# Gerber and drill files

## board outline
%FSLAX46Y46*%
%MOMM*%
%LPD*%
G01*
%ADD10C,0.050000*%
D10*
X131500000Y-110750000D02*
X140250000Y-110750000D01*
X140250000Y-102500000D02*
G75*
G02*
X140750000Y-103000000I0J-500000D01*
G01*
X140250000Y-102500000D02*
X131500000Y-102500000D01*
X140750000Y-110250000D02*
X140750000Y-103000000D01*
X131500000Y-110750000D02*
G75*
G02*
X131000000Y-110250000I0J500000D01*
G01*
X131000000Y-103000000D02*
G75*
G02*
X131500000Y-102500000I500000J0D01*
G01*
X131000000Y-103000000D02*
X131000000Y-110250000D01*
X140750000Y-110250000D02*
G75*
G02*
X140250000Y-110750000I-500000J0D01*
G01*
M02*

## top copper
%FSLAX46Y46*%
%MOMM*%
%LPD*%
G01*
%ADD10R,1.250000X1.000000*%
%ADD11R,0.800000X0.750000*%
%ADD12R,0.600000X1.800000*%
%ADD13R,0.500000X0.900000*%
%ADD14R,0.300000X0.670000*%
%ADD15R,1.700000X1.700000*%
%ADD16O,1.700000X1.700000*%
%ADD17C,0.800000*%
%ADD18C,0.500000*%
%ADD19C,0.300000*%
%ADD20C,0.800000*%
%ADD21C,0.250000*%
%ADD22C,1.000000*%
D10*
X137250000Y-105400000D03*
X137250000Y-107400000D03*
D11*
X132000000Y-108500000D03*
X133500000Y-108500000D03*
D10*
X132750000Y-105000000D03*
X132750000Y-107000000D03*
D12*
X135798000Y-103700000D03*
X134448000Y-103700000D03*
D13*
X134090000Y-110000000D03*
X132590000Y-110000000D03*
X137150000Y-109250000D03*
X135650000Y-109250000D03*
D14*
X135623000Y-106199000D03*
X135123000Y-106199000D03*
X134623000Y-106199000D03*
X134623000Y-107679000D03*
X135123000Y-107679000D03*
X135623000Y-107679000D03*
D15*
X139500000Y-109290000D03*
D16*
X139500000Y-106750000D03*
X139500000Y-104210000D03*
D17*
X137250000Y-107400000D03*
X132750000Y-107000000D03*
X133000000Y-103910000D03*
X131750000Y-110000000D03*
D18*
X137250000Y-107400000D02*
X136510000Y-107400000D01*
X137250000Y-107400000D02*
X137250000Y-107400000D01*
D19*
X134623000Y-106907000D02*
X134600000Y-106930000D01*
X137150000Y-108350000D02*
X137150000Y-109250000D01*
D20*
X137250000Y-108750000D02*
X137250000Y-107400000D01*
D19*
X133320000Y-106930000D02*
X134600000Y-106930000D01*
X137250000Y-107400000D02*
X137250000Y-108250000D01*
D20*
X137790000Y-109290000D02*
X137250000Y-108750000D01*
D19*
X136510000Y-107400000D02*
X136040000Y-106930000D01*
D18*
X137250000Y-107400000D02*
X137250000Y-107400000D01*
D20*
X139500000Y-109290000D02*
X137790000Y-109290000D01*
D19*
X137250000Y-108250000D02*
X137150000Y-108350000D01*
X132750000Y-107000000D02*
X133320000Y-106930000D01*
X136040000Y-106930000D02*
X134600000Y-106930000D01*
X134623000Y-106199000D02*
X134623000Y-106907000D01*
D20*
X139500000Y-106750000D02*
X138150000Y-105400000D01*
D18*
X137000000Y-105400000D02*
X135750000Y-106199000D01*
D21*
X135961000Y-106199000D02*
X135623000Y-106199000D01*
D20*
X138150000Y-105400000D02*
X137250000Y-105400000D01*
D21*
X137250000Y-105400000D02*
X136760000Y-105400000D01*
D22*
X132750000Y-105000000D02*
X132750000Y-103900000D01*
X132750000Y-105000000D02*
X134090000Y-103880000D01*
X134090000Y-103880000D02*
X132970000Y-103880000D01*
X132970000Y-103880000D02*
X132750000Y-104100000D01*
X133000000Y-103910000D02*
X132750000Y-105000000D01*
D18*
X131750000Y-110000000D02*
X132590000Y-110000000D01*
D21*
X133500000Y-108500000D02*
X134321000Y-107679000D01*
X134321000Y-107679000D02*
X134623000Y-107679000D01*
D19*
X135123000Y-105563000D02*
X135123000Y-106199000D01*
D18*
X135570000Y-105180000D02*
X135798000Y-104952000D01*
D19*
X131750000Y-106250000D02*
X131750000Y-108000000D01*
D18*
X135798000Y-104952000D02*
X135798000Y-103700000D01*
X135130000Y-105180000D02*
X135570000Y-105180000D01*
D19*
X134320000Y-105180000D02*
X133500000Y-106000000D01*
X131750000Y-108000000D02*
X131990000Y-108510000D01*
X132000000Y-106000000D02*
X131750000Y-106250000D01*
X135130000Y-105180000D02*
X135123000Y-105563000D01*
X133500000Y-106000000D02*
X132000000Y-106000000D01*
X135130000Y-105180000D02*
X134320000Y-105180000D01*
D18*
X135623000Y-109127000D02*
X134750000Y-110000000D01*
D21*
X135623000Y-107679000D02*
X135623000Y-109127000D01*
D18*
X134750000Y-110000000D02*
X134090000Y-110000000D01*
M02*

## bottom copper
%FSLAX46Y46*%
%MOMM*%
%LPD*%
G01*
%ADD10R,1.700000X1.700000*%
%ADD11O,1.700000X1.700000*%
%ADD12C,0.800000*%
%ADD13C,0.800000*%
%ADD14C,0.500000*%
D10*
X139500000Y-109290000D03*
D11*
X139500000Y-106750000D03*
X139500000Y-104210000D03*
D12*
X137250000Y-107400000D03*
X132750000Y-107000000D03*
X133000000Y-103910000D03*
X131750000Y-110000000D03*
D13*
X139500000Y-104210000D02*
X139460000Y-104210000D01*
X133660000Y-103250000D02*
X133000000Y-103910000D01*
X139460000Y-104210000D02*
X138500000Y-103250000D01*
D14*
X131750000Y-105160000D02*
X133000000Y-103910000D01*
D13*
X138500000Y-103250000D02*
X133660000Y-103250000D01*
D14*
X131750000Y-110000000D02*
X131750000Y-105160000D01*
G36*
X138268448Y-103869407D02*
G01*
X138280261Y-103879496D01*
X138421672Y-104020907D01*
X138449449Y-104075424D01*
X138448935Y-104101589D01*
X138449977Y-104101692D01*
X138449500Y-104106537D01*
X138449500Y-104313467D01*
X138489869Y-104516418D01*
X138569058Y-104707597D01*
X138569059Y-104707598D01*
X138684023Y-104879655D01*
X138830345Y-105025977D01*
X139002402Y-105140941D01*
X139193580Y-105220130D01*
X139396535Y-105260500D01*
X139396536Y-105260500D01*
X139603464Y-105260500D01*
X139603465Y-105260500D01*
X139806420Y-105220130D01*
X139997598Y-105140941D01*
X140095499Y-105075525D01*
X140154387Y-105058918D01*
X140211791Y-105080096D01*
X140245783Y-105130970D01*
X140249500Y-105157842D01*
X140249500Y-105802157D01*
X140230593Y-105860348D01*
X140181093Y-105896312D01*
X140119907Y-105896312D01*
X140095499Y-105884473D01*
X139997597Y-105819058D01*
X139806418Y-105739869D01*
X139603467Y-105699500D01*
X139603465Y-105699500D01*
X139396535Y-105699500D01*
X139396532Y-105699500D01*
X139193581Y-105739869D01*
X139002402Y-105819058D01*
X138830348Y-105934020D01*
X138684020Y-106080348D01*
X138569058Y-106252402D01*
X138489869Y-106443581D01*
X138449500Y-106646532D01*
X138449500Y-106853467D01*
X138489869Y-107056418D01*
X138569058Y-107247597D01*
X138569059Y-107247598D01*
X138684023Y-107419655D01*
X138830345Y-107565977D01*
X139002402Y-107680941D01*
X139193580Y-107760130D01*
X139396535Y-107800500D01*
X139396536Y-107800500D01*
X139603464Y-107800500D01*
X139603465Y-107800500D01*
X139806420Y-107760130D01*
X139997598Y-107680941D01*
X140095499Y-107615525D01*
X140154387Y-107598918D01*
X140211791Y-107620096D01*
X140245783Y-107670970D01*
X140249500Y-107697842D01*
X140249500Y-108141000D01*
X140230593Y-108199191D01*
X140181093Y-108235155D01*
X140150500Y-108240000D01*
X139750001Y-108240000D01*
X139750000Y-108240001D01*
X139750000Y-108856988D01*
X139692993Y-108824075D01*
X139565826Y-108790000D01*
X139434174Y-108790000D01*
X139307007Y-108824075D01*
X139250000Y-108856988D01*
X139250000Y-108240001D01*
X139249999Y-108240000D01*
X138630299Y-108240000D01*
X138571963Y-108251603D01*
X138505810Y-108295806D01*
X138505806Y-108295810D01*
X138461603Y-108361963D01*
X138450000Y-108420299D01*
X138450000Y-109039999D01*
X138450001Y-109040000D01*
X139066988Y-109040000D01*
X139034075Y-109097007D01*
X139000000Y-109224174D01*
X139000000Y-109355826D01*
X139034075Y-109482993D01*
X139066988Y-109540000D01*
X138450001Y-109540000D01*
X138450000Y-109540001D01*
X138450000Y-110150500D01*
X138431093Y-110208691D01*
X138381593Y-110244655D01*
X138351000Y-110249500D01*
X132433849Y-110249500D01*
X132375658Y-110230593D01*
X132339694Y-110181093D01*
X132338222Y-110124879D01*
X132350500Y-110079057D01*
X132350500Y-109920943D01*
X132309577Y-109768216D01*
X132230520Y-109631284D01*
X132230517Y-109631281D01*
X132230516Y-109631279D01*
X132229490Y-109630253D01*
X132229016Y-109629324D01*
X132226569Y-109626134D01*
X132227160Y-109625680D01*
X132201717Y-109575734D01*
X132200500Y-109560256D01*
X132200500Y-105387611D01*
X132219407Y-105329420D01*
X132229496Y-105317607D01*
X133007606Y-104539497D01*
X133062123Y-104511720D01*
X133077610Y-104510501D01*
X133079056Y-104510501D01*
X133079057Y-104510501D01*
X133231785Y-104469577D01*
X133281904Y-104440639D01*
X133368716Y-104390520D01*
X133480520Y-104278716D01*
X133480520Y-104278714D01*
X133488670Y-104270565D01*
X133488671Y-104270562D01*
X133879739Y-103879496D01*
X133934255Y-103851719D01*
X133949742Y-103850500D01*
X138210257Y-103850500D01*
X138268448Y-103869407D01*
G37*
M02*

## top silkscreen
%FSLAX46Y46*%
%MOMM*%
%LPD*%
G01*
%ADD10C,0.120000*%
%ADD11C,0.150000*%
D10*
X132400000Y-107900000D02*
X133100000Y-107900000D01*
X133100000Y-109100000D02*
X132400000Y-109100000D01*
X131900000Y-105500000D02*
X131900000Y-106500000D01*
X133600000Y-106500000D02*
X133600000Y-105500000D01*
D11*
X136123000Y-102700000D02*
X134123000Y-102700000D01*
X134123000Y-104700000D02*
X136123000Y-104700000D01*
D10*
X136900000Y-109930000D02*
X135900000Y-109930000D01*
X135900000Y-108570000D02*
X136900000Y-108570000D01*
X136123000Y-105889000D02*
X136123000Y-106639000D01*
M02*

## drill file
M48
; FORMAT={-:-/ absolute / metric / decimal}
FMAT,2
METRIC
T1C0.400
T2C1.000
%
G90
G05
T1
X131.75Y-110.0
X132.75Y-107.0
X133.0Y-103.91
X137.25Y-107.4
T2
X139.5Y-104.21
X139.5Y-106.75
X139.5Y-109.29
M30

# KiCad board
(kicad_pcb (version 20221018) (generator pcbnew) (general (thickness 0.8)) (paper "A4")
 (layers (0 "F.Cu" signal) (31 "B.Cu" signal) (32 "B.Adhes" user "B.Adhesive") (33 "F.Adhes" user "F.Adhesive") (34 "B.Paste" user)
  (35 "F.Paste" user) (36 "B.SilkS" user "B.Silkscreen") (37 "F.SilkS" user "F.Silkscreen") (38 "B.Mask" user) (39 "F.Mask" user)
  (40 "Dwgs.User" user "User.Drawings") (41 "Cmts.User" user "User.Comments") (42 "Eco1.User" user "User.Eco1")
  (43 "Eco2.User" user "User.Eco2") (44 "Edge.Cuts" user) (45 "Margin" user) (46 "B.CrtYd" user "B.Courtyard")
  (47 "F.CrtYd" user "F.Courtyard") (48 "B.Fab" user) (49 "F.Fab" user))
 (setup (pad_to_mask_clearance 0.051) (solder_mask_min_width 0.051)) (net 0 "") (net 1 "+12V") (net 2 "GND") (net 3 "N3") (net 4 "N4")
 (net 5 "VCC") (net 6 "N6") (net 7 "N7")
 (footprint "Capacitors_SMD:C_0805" (layer "F.Cu") (at 137.25 106.4 -90)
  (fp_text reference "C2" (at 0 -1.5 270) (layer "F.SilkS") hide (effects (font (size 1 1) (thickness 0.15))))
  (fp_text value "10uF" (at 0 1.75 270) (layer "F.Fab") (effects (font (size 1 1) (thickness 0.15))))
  (pad "1" smd rect (at -1 0 270) (size 1 1.25) (layers "F.Cu" "F.Paste" "F.Mask") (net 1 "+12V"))
  (pad "2" smd rect (at 1 0 270) (size 1 1.25) (layers "F.Cu" "F.Paste" "F.Mask") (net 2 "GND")))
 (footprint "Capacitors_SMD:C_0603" (layer "F.Cu") (at 132.75 108.5)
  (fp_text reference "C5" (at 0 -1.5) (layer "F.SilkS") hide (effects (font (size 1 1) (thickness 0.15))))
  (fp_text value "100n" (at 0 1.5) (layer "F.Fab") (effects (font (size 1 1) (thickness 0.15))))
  (fp_line (start -0.35 -0.6) (end 0.35 -0.6) (stroke (width 0.12) (type solid)) (layer "F.SilkS"))
  (fp_line (start 0.35 0.6) (end -0.35 0.6) (stroke (width 0.12) (type solid)) (layer "F.SilkS"))
  (pad "1" smd rect (at -0.75 0) (size 0.8 0.75) (layers "F.Cu" "F.Paste" "F.Mask") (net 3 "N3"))
  (pad "2" smd rect (at 0.75 0) (size 0.8 0.75) (layers "F.Cu" "F.Paste" "F.Mask") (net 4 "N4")))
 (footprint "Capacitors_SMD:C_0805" (layer "F.Cu") (at 132.75 106 -90)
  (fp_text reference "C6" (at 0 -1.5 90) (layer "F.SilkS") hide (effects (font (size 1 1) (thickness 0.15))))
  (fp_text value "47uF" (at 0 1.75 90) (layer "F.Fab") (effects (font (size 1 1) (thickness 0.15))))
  (fp_line (start -0.5 0.85) (end 0.5 0.85) (stroke (width 0.12) (type solid)) (layer "F.SilkS"))
  (fp_line (start 0.5 -0.85) (end -0.5 -0.85) (stroke (width 0.12) (type solid)) (layer "F.SilkS"))
  (pad "1" smd rect (at -1 0 270) (size 1 1.25) (layers "F.Cu" "F.Paste" "F.Mask") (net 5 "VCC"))
  (pad "2" smd rect (at 1 0 270) (size 1 1.25) (layers "F.Cu" "F.Paste" "F.Mask") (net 2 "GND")))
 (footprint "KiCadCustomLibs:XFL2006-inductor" (layer "F.Cu") (at 135.123 103.7 180)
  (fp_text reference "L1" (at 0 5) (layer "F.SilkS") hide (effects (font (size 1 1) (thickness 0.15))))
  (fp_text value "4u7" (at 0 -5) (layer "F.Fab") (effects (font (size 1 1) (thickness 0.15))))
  (fp_line (start -1 1) (end 1 1) (stroke (width 0.15) (type solid)) (layer "F.SilkS"))
  (fp_line (start 1 -1) (end -1 -1) (stroke (width 0.15) (type solid)) (layer "F.SilkS"))
  (pad "1" smd rect (at -0.675 0 180) (size 0.6 1.8) (layers "F.Cu" "F.Paste" "F.Mask") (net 3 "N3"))
  (pad "2" smd rect (at 0.675 0 180) (size 0.6 1.8) (layers "F.Cu" "F.Paste" "F.Mask") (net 5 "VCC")))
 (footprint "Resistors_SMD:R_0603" (layer "F.Cu") (at 133.34 110 180)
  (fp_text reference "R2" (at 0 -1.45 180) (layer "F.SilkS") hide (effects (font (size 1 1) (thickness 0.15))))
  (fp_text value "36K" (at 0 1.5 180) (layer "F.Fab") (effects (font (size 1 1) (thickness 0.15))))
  (pad "1" smd rect (at -0.75 0 180) (size 0.5 0.9) (layers "F.Cu" "F.Paste" "F.Mask") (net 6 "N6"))
  (pad "2" smd rect (at 0.75 0 180) (size 0.5 0.9) (layers "F.Cu" "F.Paste" "F.Mask") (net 5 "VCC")))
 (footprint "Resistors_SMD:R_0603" (layer "F.Cu") (at 136.4 109.25 180)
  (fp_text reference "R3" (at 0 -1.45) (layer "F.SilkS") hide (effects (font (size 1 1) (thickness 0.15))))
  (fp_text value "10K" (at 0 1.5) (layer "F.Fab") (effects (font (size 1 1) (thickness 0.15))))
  (fp_line (start -0.5 -0.68) (end 0.5 -0.68) (stroke (width 0.12) (type solid)) (layer "F.SilkS"))
  (fp_line (start 0.5 0.68) (end -0.5 0.68) (stroke (width 0.12) (type solid)) (layer "F.SilkS"))
  (pad "1" smd rect (at -0.75 0 180) (size 0.5 0.9) (layers "F.Cu" "F.Paste" "F.Mask") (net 2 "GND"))
  (pad "2" smd rect (at 0.75 0 180) (size 0.5 0.9) (layers "F.Cu" "F.Paste" "F.Mask") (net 6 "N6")))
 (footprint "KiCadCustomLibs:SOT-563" (layer "F.Cu") (at 135.123 106.939 -90)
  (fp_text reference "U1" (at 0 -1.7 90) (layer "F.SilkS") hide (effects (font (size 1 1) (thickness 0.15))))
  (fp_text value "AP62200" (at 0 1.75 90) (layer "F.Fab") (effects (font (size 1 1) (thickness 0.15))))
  (fp_line (start -1.05 -1) (end -0.3 -1) (stroke (width 0.12) (type solid)) (layer "F.SilkS"))
  (pad "1" smd rect (at -0.74 -0.5 270) (size 0.67 0.3) (layers "F.Cu" "F.Paste" "F.Mask") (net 1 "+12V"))
  (pad "2" smd rect (at -0.74 0 270) (size 0.67 0.3) (layers "F.Cu" "F.Paste" "F.Mask") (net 3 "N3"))
  (pad "3" smd rect (at -0.74 0.5 270) (size 0.67 0.3) (layers "F.Cu" "F.Paste" "F.Mask") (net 2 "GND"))
  (pad "4" smd rect (at 0.74 0.5 270) (size 0.67 0.3) (layers "F.Cu" "F.Paste" "F.Mask") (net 4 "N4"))
  (pad "5" smd rect (at 0.74 0 270) (size 0.67 0.3) (layers "F.Cu" "F.Paste" "F.Mask") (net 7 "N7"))
  (pad "6" smd rect (at 0.74 -0.5 270) (size 0.67 0.3) (layers "F.Cu" "F.Paste" "F.Mask") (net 6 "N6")))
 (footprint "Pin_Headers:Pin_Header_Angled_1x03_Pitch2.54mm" (layer "B.Cu") (at 139.5 109.29)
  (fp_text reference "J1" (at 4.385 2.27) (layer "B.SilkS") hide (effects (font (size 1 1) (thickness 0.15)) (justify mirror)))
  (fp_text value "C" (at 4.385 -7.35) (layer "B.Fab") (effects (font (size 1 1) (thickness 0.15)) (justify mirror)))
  (pad "1" thru_hole rect (at 0 0) (size 1.7 1.7) (drill 1) (layers "*.Cu" "*.Mask") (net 2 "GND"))
  (pad "2" thru_hole oval (at 0 -2.54) (size 1.7 1.7) (drill 1) (layers "*.Cu" "*.Mask") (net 1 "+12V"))
  (pad "3" thru_hole oval (at 0 -5.08) (size 1.7 1.7) (drill 1) (layers "*.Cu" "*.Mask") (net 5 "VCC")))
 (gr_line (start 131.5 110.75) (end 140.25 110.75) (stroke (width 0.05) (type solid)) (layer "Edge.Cuts"))
 (gr_arc (start 140.25 102.5) (mid 140.603553 102.646447) (end 140.75 103) (stroke (width 0.05) (type solid)) (layer "Edge.Cuts"))
 (gr_line (start 140.25 102.5) (end 131.5 102.5) (stroke (width 0.05) (type solid)) (layer "Edge.Cuts"))
 (gr_line (start 140.75 110.25) (end 140.75 103) (stroke (width 0.05) (type solid)) (layer "Edge.Cuts"))
 (gr_arc (start 131.5 110.75) (mid 131.146447 110.603553) (end 131 110.25) (stroke (width 0.05) (type solid)) (layer "Edge.Cuts"))
 (gr_arc (start 131 103) (mid 131.146447 102.646447) (end 131.5 102.5) (stroke (width 0.05) (type solid)) (layer "Edge.Cuts"))
 (gr_line (start 131 103) (end 131 110.25) (stroke (width 0.05) (type solid)) (layer "Edge.Cuts"))
 (gr_arc (start 140.75 110.25) (mid 140.603553 110.603553) (end 140.25 110.75) (stroke (width 0.05) (type solid)) (layer "Edge.Cuts"))
 (segment (start 137.25 107.4) (end 136.51 107.4) (width 0.5) (layer "F.Cu") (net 2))
 (segment (start 137.25 107.4) (end 137.25 107.4) (width 0.5) (layer "F.Cu") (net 2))
 (segment (start 134.623 106.907) (end 134.6 106.93) (width 0.3) (layer "F.Cu") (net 2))
 (segment (start 137.15 108.35) (end 137.15 109.25) (width 0.3) (layer "F.Cu") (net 2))
 (segment (start 137.25 108.75) (end 137.25 107.4) (width 0.8) (layer "F.Cu") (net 2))
 (segment (start 133.32 106.93) (end 134.6 106.93) (width 0.3) (layer "F.Cu") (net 2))
 (segment (start 137.25 107.4) (end 137.25 108.25) (width 0.3) (layer "F.Cu") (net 2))
 (segment (start 137.79 109.29) (end 137.25 108.75) (width 0.8) (layer "F.Cu") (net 2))
 (segment (start 136.51 107.4) (end 136.04 106.93) (width 0.3) (layer "F.Cu") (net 2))
 (segment (start 137.25 107.4) (end 137.25 107.4) (width 0.5) (layer "F.Cu") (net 2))
 (segment (start 139.5 109.29) (end 137.79 109.29) (width 0.8) (layer "F.Cu") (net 2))
 (segment (start 137.25 108.25) (end 137.15 108.35) (width 0.3) (layer "F.Cu") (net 2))
 (segment (start 132.75 107) (end 133.32 106.93) (width 0.3) (layer "F.Cu") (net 2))
 (segment (start 136.04 106.93) (end 134.6 106.93) (width 0.3) (layer "F.Cu") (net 2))
 (segment (start 134.623 106.199) (end 134.623 106.907) (width 0.3) (layer "F.Cu") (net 2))
 (via (at 137.25 107.4) (size 0.8) (drill 0.4) (layers "F.Cu" "B.Cu") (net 2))
 (via (at 132.75 107) (size 0.8) (drill 0.4) (layers "F.Cu" "B.Cu") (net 2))
 (segment (start 139.5 106.75) (end 138.15 105.4) (width 0.8) (layer "F.Cu") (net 1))
 (segment (start 137 105.4) (end 135.75 106.199) (width 0.5) (layer "F.Cu") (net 1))
 (segment (start 135.961 106.199) (end 135.623 106.199) (width 0.25) (layer "F.Cu") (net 1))
 (segment (start 138.15 105.4) (end 137.25 105.4) (width 0.8) (layer "F.Cu") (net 1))
 (segment (start 137.25 105.4) (end 136.76 105.4) (width 0.25) (layer "F.Cu") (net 1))
 (segment (start 132.75 105) (end 132.75 103.9) (width 1) (layer "F.Cu") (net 5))
 (segment (start 132.75 105) (end 134.09 103.88) (width 1) (layer "F.Cu") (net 5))
 (segment (start 134.09 103.88) (end 132.97 103.88) (width 1) (layer "F.Cu") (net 5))
 (segment (start 132.97 103.88) (end 132.75 104.1) (width 1) (layer "F.Cu") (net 5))
 (segment (start 133 103.91) (end 132.75 105) (width 1) (layer "F.Cu") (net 5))
 (segment (start 131.75 110) (end 132.59 110) (width 0.5) (layer "F.Cu") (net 5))
 (via (at 133 103.91) (size 0.8) (drill 0.4) (layers "F.Cu" "B.Cu") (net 5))
 (via (at 131.75 110) (size 0.8) (drill 0.4) (layers "F.Cu" "B.Cu") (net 5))
 (segment (start 139.5 104.21) (end 139.46 104.21) (width 0.8) (layer "B.Cu") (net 5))
 (segment (start 133.66 103.25) (end 133 103.91) (width 0.8) (layer "B.Cu") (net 5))
 (segment (start 139.46 104.21) (end 138.5 103.25) (width 0.8) (layer "B.Cu") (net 5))
 (segment (start 131.75 105.16) (end 133 103.91) (width 0.5) (layer "B.Cu") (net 5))
 (segment (start 138.5 103.25) (end 133.66 103.25) (width 0.8) (layer "B.Cu") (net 5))
 (segment (start 131.75 110) (end 131.75 105.16) (width 0.5) (layer "B.Cu") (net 5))
 (segment (start 133.5 108.5) (end 134.321 107.679) (width 0.25) (layer "F.Cu") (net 4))
 (segment (start 134.321 107.679) (end 134.623 107.679) (width 0.25) (layer "F.Cu") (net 4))
 (segment (start 135.123 105.563) (end 135.123 106.199) (width 0.3) (layer "F.Cu") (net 3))
 (segment (start 135.57 105.18) (end 135.798 104.952) (width 0.5) (layer "F.Cu") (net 3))
 (segment (start 131.75 106.25) (end 131.75 108) (width 0.3) (layer "F.Cu") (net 3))
 (segment (start 135.798 104.952) (end 135.798 103.7) (width 0.5) (layer "F.Cu") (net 3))
 (segment (start 135.13 105.18) (end 135.57 105.18) (width 0.5) (layer "F.Cu") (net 3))
 (segment (start 134.32 105.18) (end 133.5 106) (width 0.3) (layer "F.Cu") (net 3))
 (segment (start 131.75 108) (end 131.99 108.51) (width 0.3) (layer "F.Cu") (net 3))
 (segment (start 132 106) (end 131.75 106.25) (width 0.3) (layer "F.Cu") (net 3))
 (segment (start 135.13 105.18) (end 135.123 105.563) (width 0.3) (layer "F.Cu") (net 3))
 (segment (start 133.5 106) (end 132 106) (width 0.3) (layer "F.Cu") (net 3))
 (segment (start 135.13 105.18) (end 134.32 105.18) (width 0.3) (layer "F.Cu") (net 3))
 (segment (start 135.623 109.127) (end 134.75 110) (width 0.5) (layer "F.Cu") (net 6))
 (segment (start 135.623 107.679) (end 135.623 109.127) (width 0.25) (layer "F.Cu") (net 6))
 (segment (start 134.75 110) (end 134.09 110) (width 0.5) (layer "F.Cu") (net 6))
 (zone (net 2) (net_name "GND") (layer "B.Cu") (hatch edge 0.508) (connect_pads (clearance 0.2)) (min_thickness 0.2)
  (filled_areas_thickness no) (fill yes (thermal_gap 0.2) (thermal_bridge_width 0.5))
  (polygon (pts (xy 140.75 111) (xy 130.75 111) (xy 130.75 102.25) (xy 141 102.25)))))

